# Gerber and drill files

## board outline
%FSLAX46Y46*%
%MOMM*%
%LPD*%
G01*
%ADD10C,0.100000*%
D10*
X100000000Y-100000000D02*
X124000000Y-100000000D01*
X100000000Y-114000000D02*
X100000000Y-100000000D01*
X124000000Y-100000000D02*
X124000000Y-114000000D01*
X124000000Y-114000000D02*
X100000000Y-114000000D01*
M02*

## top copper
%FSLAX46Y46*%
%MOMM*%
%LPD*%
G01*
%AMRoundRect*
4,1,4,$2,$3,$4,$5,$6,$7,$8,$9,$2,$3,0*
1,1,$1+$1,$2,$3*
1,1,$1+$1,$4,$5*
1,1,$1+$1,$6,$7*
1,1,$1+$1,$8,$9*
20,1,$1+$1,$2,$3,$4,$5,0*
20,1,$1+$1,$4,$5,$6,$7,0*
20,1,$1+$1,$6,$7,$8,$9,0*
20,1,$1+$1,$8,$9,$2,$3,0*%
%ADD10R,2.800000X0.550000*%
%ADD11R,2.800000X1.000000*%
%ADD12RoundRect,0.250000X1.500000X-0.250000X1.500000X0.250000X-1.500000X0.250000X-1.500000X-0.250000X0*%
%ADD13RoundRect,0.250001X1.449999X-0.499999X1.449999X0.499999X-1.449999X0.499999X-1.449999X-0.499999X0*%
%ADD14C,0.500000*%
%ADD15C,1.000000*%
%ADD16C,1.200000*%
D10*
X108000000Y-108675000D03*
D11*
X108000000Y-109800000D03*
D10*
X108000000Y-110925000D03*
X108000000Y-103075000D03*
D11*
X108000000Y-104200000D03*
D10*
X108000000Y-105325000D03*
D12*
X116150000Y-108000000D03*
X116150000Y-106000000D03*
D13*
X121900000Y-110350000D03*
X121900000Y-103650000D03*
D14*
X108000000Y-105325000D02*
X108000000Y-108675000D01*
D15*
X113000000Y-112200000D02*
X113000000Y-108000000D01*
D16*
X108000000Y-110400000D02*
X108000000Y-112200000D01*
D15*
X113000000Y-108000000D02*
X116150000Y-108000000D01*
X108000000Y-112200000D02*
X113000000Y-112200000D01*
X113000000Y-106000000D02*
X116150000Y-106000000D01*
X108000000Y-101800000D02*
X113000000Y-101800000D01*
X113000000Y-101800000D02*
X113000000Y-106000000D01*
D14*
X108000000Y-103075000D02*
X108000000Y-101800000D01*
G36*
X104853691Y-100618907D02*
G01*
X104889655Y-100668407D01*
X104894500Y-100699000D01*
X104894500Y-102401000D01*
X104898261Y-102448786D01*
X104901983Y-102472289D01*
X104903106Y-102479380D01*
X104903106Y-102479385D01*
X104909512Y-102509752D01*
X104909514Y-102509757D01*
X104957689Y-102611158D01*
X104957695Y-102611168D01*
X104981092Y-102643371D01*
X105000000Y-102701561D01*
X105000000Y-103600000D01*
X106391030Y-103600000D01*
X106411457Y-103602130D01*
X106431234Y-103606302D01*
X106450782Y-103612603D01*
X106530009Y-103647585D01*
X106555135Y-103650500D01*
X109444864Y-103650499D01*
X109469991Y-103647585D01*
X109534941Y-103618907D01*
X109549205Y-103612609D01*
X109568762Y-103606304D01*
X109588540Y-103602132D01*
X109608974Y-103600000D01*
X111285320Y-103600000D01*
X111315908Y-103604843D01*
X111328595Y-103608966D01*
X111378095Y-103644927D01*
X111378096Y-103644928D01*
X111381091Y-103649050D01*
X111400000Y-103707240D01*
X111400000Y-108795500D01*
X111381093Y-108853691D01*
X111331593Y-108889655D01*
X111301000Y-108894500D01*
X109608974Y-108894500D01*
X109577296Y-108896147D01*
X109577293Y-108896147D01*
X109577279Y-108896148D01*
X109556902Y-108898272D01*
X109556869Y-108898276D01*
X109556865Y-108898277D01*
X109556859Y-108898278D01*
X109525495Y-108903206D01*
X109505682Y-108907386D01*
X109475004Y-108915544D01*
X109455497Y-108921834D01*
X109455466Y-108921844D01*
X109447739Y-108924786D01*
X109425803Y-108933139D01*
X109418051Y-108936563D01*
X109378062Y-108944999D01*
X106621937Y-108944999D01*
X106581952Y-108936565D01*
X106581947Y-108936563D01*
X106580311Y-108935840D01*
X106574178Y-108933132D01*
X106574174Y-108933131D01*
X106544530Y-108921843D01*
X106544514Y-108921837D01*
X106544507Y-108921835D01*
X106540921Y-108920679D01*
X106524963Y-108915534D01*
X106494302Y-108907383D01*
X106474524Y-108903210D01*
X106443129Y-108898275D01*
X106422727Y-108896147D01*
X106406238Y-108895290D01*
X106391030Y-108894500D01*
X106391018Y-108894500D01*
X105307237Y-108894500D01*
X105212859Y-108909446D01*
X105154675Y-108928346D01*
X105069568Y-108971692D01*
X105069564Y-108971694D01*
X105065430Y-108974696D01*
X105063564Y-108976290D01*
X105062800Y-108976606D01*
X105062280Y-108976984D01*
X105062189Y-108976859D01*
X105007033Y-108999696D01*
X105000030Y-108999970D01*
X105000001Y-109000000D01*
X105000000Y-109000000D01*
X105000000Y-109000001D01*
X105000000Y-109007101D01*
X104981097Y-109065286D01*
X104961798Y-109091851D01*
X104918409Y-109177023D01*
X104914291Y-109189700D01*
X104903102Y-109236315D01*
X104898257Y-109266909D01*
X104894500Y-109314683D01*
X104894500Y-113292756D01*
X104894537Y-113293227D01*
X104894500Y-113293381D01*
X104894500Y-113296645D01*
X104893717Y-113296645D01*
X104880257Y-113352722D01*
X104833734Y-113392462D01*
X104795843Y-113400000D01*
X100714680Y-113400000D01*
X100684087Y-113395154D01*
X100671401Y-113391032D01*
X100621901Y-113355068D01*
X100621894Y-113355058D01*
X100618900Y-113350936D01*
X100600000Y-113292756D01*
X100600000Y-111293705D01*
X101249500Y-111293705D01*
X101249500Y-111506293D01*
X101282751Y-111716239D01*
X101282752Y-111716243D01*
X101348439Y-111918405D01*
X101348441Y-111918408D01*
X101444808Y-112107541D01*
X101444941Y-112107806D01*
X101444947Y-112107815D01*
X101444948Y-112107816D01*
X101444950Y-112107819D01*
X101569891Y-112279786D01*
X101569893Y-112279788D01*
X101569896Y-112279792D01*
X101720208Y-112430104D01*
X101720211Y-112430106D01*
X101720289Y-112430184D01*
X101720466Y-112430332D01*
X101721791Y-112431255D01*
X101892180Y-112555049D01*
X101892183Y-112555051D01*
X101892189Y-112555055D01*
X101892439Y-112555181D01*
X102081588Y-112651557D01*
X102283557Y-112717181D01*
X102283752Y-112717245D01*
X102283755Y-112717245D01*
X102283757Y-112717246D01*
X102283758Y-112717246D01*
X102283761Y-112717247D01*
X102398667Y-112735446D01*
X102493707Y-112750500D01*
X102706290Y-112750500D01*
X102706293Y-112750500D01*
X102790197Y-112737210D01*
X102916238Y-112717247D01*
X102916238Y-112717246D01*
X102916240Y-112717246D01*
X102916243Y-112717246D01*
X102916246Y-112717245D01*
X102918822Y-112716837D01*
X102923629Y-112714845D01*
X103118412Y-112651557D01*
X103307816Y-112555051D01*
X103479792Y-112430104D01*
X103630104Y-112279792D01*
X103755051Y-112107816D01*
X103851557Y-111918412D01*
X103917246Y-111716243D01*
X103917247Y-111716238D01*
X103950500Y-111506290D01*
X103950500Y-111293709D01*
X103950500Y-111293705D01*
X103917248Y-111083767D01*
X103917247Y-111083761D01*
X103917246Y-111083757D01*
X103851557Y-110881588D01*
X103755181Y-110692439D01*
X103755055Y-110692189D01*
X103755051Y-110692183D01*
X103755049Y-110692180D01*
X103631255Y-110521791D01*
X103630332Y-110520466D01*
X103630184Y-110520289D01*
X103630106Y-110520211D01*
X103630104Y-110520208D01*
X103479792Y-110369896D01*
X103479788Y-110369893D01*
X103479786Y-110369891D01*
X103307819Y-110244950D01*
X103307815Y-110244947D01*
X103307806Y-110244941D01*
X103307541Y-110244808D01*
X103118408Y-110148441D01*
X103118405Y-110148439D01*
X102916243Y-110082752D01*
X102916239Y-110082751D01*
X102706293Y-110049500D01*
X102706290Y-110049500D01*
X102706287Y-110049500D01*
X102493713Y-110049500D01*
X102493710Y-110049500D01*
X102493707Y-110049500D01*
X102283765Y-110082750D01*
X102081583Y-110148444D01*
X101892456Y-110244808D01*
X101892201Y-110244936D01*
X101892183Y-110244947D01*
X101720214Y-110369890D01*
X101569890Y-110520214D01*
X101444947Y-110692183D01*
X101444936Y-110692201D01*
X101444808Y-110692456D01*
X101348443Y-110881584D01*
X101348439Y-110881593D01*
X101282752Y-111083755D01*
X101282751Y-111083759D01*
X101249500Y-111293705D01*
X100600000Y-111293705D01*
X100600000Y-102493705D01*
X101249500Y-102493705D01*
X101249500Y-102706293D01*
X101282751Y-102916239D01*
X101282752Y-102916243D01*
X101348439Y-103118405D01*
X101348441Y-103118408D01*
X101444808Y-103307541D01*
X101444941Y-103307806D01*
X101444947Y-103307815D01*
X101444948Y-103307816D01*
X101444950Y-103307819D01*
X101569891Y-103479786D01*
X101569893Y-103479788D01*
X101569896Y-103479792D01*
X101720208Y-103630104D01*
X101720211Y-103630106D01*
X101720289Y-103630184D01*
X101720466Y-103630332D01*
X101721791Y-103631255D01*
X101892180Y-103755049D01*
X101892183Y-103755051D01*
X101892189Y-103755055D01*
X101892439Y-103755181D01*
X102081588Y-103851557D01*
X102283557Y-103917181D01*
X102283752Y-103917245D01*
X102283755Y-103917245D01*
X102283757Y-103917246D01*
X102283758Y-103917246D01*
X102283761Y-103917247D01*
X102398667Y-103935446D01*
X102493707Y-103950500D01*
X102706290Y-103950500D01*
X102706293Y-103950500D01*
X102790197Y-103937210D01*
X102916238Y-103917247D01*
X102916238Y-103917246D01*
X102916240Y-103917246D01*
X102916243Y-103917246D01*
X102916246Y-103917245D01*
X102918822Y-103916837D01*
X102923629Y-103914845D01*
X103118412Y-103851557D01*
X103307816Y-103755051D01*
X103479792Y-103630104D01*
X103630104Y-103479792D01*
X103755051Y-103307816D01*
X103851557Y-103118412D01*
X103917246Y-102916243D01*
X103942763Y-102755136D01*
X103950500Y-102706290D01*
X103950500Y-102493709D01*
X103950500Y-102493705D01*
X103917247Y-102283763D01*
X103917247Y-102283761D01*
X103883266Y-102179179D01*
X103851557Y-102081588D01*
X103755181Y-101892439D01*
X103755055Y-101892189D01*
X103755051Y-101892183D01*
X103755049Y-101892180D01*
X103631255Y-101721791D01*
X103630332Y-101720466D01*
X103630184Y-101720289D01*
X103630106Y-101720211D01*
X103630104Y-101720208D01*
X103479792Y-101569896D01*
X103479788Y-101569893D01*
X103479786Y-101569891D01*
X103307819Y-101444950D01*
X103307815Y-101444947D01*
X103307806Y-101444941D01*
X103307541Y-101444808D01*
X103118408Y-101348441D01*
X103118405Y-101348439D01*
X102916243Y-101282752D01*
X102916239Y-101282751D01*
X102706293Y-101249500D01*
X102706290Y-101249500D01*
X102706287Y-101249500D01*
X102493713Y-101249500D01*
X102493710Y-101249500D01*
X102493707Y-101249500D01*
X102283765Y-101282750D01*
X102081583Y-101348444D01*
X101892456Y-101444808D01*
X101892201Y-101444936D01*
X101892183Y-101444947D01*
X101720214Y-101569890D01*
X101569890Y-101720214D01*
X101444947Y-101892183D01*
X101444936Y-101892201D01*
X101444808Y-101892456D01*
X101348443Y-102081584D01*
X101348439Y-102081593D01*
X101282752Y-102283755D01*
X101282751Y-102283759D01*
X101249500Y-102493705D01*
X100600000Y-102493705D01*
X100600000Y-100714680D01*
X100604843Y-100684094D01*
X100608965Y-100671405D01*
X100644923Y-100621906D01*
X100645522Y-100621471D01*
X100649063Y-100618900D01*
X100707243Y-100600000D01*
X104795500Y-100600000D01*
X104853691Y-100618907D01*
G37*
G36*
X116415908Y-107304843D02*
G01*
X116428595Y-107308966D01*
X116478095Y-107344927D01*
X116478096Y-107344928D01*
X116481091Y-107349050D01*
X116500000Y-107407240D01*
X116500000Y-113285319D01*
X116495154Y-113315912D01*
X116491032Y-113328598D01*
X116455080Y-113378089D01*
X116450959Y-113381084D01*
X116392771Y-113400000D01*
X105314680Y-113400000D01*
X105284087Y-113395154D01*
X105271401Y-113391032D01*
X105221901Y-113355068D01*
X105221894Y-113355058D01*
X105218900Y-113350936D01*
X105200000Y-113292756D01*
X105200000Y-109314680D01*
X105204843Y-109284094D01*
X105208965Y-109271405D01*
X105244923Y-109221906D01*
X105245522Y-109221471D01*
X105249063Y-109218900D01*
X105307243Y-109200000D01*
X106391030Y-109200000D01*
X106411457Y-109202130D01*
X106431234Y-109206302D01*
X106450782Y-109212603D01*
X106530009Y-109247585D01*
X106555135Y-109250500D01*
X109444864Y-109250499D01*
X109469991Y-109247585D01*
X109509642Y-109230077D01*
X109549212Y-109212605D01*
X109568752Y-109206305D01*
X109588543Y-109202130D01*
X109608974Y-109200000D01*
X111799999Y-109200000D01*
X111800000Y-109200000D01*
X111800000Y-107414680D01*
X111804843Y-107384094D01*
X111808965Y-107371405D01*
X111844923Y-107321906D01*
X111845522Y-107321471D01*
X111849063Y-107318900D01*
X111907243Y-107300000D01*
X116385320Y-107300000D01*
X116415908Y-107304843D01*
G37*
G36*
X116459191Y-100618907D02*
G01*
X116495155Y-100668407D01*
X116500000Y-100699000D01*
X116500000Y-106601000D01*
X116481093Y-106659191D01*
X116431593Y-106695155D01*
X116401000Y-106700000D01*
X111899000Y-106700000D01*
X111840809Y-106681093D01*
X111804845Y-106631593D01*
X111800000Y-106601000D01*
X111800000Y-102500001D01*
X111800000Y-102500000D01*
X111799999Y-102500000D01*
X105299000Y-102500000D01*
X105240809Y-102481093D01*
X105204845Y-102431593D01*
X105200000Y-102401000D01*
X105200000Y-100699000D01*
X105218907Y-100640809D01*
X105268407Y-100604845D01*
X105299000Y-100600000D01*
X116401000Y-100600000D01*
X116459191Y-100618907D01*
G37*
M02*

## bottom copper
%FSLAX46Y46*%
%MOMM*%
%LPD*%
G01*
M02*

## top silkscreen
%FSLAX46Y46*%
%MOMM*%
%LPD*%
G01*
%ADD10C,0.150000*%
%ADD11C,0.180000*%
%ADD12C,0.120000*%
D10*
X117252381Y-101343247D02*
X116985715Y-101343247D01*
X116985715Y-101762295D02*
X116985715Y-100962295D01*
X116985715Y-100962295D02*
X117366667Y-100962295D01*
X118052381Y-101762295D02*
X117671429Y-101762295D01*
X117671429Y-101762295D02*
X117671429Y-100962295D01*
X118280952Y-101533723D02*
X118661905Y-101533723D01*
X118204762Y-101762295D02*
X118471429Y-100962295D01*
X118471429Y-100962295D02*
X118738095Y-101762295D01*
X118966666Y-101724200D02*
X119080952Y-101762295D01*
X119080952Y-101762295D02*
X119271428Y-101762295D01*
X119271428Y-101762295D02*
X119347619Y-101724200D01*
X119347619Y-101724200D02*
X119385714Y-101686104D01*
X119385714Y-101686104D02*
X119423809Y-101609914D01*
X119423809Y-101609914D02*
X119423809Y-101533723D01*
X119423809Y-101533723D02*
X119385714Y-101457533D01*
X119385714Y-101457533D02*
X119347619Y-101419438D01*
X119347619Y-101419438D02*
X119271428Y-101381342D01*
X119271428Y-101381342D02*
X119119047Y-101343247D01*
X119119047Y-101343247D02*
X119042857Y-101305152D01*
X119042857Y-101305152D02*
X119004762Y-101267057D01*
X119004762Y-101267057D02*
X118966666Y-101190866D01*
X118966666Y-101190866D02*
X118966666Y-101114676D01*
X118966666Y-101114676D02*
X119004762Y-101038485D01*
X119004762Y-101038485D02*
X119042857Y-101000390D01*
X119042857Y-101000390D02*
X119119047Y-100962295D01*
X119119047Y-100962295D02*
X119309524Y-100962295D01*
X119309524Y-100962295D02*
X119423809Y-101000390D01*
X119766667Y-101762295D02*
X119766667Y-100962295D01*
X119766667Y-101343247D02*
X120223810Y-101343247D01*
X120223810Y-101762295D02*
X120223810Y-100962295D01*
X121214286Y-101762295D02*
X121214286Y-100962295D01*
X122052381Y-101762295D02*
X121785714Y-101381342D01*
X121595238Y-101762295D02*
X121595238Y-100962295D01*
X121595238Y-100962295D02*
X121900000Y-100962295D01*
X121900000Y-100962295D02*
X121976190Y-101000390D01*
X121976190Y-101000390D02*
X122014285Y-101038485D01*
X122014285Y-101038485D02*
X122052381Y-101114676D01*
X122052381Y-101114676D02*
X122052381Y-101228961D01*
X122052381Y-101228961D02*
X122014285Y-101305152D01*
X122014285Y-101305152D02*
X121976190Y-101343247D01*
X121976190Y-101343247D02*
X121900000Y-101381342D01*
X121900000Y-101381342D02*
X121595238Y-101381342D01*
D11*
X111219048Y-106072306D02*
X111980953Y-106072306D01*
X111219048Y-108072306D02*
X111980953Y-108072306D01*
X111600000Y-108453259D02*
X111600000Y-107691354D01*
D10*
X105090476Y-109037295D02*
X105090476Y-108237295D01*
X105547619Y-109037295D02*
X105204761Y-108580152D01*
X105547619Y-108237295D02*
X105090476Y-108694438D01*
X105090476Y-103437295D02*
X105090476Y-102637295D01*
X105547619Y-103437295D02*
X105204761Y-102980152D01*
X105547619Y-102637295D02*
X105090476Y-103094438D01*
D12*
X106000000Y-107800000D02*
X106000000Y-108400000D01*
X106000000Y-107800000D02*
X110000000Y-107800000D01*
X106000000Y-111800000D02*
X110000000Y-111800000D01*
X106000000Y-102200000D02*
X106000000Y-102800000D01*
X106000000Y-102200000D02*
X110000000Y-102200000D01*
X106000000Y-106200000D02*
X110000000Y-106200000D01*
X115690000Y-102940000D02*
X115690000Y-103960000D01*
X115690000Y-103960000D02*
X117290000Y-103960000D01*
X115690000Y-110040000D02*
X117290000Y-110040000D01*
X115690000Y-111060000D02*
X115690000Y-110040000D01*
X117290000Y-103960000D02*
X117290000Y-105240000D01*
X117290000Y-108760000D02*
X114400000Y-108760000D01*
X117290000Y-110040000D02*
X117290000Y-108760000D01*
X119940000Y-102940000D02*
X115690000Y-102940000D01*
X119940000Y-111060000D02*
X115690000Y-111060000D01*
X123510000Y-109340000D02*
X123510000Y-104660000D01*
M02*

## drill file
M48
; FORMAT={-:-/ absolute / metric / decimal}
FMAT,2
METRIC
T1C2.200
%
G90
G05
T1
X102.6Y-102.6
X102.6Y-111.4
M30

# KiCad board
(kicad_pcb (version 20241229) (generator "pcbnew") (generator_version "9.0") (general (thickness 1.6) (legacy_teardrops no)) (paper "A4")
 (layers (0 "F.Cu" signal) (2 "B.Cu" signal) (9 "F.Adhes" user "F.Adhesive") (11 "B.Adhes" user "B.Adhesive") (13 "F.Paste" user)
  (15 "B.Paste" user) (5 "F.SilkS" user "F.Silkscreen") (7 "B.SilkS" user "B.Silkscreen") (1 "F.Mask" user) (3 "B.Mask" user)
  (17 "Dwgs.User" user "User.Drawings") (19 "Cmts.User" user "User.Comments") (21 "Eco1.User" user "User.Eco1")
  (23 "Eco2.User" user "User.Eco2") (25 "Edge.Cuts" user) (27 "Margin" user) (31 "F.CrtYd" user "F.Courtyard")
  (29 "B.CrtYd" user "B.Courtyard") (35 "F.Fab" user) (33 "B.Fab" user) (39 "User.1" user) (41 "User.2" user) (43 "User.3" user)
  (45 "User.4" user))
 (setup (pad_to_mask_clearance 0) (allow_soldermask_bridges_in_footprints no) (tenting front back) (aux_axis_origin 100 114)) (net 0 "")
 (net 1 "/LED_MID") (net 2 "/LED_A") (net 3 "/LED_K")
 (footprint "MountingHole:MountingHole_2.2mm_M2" (layer "F.Cu") (at 102.6 111.4)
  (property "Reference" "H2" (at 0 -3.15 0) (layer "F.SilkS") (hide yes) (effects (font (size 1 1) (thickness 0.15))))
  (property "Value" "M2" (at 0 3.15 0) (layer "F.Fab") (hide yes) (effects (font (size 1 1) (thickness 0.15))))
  (pad "" np_thru_hole circle (at 0 0) (size 2.2 2.2) (drill 2.2) (layers "*.Cu" "*.Mask")))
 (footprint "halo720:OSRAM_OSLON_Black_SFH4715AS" (layer "F.Cu") (at 108 109.8)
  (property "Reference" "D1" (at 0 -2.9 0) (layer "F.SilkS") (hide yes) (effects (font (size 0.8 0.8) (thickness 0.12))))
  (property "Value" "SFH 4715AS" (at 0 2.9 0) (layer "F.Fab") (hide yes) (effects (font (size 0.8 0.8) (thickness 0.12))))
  (fp_line (start -2 -2) (end -2 -1.4) (stroke (width 0.12) (type solid)) (layer "F.SilkS"))
  (fp_line (start -2 -2) (end 2 -2) (stroke (width 0.12) (type solid)) (layer "F.SilkS"))
  (fp_line (start -2 2) (end 2 2) (stroke (width 0.12) (type solid)) (layer "F.SilkS"))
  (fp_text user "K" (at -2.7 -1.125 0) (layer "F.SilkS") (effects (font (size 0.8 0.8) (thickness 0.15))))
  (pad "1" smd rect (at 0 -1.125) (size 2.8 0.55) (layers "F.Cu" "F.Mask" "F.Paste") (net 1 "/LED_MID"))
  (pad "2" smd rect (at 0 0) (size 2.8 1) (layers "F.Cu" "F.Mask" "F.Paste") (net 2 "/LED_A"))
  (pad "2" smd rect (at 0 1.125) (size 2.8 0.55) (layers "F.Cu" "F.Mask" "F.Paste") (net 2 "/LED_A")))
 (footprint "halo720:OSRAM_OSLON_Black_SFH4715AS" (layer "F.Cu") (at 108 104.2)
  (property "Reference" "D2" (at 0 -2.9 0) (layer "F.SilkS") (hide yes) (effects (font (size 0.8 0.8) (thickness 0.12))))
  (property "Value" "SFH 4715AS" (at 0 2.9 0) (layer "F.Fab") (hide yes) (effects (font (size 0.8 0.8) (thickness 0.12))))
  (fp_line (start -2 -2) (end -2 -1.4) (stroke (width 0.12) (type solid)) (layer "F.SilkS"))
  (fp_line (start -2 -2) (end 2 -2) (stroke (width 0.12) (type solid)) (layer "F.SilkS"))
  (fp_line (start -2 2) (end 2 2) (stroke (width 0.12) (type solid)) (layer "F.SilkS"))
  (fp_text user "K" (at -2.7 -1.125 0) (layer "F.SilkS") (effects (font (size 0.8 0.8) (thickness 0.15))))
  (pad "1" smd rect (at 0 -1.125) (size 2.8 0.55) (layers "F.Cu" "F.Mask" "F.Paste") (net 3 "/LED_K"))
  (pad "2" smd rect (at 0 0) (size 2.8 1) (layers "F.Cu" "F.Mask" "F.Paste") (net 1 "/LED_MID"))
  (pad "2" smd rect (at 0 1.125) (size 2.8 0.55) (layers "F.Cu" "F.Mask" "F.Paste") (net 1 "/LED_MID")))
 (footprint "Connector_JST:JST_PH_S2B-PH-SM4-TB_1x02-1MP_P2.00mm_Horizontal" (layer "F.Cu") (at 119 107 90)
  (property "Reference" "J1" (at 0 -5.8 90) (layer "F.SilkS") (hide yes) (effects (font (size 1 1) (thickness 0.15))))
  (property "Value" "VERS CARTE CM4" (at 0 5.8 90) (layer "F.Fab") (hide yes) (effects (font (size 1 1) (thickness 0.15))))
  (fp_line (start 4.06 -3.31) (end 3.04 -3.31) (stroke (width 0.12) (type solid)) (layer "F.SilkS"))
  (fp_line (start 3.04 -3.31) (end 3.04 -1.71) (stroke (width 0.12) (type solid)) (layer "F.SilkS"))
  (fp_line (start -3.04 -3.31) (end -3.04 -1.71) (stroke (width 0.12) (type solid)) (layer "F.SilkS"))
  (fp_line (start -4.06 -3.31) (end -3.04 -3.31) (stroke (width 0.12) (type solid)) (layer "F.SilkS"))
  (fp_line (start 3.04 -1.71) (end 1.76 -1.71) (stroke (width 0.12) (type solid)) (layer "F.SilkS"))
  (fp_line (start -1.76 -1.71) (end -1.76 -4.6) (stroke (width 0.12) (type solid)) (layer "F.SilkS"))
  (fp_line (start -3.04 -1.71) (end -1.76 -1.71) (stroke (width 0.12) (type solid)) (layer "F.SilkS"))
  (fp_line (start 4.06 0.94) (end 4.06 -3.31) (stroke (width 0.12) (type solid)) (layer "F.SilkS"))
  (fp_line (start -4.06 0.94) (end -4.06 -3.31) (stroke (width 0.12) (type solid)) (layer "F.SilkS"))
  (fp_line (start -2.34 4.51) (end 2.34 4.51) (stroke (width 0.12) (type solid)) (layer "F.SilkS"))
  (pad "1" smd roundrect (at -1 -2.85 90) (size 1 3.5) (layers "F.Cu" "F.Mask" "F.Paste") (roundrect_rratio 0.25) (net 2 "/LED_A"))
  (pad "2" smd roundrect (at 1 -2.85 90) (size 1 3.5) (layers "F.Cu" "F.Mask" "F.Paste") (roundrect_rratio 0.25) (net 3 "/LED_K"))
  (pad "MP" smd roundrect (at -3.35 2.9 90) (size 1.5 3.4) (layers "F.Cu" "F.Mask" "F.Paste") (roundrect_rratio 0.166667))
  (pad "MP" smd roundrect (at 3.35 2.9 90) (size 1.5 3.4) (layers "F.Cu" "F.Mask" "F.Paste") (roundrect_rratio 0.166667)))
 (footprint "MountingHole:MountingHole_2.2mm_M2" (layer "F.Cu") (at 102.6 102.6)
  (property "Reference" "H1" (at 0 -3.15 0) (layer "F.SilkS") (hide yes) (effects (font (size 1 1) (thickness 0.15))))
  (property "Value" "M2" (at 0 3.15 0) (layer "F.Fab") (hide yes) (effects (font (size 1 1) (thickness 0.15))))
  (pad "" np_thru_hole circle (at 0 0) (size 2.2 2.2) (drill 2.2) (layers "*.Cu" "*.Mask")))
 (gr_line (start 100 100) (end 124 100) (stroke (width 0.1) (type default)) (layer "Edge.Cuts"))
 (gr_line (start 100 114) (end 100 100) (stroke (width 0.1) (type default)) (layer "Edge.Cuts"))
 (gr_line (start 124 100) (end 124 114) (stroke (width 0.1) (type default)) (layer "Edge.Cuts"))
 (gr_line (start 124 114) (end 100 114) (stroke (width 0.1) (type default)) (layer "Edge.Cuts"))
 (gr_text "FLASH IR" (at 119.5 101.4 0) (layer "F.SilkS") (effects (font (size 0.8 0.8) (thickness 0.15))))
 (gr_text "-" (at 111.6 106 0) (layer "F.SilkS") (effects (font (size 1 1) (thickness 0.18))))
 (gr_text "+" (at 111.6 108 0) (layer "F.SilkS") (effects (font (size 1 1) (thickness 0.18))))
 (segment (start 108 105.325) (end 108 108.675) (width 0.5) (layer "F.Cu") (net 1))
 (segment (start 113 112.2) (end 113 108) (width 1) (layer "F.Cu") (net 2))
 (segment (start 108 110.4) (end 108 112.2) (width 1.2) (layer "F.Cu") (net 2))
 (segment (start 113 108) (end 116.15 108) (width 1) (layer "F.Cu") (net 2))
 (segment (start 108 112.2) (end 113 112.2) (width 1) (layer "F.Cu") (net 2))
 (segment (start 113 106) (end 116.15 106) (width 1) (layer "F.Cu") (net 3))
 (segment (start 108 101.8) (end 113 101.8) (width 1) (layer "F.Cu") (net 3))
 (segment (start 113 101.8) (end 113 106) (width 1) (layer "F.Cu") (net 3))
 (segment (start 108 103.075) (end 108 101.8) (width 0.5) (layer "F.Cu") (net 3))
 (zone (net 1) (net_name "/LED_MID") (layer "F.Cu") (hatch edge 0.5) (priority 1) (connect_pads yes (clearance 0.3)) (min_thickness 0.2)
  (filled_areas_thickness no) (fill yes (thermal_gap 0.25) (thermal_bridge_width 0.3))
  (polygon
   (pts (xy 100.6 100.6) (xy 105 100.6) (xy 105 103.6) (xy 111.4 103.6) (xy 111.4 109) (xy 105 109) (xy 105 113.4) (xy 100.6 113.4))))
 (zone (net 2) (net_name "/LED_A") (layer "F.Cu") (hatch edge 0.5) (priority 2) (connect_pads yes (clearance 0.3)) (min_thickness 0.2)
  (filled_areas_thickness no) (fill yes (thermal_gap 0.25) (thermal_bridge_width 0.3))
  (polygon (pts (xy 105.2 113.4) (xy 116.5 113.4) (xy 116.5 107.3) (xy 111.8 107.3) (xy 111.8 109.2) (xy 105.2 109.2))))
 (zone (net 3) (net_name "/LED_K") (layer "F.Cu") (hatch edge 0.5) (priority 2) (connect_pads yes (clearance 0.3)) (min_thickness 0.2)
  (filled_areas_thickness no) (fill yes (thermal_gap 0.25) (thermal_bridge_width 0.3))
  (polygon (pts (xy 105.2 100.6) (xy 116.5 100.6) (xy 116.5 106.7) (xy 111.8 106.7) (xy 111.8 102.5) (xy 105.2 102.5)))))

